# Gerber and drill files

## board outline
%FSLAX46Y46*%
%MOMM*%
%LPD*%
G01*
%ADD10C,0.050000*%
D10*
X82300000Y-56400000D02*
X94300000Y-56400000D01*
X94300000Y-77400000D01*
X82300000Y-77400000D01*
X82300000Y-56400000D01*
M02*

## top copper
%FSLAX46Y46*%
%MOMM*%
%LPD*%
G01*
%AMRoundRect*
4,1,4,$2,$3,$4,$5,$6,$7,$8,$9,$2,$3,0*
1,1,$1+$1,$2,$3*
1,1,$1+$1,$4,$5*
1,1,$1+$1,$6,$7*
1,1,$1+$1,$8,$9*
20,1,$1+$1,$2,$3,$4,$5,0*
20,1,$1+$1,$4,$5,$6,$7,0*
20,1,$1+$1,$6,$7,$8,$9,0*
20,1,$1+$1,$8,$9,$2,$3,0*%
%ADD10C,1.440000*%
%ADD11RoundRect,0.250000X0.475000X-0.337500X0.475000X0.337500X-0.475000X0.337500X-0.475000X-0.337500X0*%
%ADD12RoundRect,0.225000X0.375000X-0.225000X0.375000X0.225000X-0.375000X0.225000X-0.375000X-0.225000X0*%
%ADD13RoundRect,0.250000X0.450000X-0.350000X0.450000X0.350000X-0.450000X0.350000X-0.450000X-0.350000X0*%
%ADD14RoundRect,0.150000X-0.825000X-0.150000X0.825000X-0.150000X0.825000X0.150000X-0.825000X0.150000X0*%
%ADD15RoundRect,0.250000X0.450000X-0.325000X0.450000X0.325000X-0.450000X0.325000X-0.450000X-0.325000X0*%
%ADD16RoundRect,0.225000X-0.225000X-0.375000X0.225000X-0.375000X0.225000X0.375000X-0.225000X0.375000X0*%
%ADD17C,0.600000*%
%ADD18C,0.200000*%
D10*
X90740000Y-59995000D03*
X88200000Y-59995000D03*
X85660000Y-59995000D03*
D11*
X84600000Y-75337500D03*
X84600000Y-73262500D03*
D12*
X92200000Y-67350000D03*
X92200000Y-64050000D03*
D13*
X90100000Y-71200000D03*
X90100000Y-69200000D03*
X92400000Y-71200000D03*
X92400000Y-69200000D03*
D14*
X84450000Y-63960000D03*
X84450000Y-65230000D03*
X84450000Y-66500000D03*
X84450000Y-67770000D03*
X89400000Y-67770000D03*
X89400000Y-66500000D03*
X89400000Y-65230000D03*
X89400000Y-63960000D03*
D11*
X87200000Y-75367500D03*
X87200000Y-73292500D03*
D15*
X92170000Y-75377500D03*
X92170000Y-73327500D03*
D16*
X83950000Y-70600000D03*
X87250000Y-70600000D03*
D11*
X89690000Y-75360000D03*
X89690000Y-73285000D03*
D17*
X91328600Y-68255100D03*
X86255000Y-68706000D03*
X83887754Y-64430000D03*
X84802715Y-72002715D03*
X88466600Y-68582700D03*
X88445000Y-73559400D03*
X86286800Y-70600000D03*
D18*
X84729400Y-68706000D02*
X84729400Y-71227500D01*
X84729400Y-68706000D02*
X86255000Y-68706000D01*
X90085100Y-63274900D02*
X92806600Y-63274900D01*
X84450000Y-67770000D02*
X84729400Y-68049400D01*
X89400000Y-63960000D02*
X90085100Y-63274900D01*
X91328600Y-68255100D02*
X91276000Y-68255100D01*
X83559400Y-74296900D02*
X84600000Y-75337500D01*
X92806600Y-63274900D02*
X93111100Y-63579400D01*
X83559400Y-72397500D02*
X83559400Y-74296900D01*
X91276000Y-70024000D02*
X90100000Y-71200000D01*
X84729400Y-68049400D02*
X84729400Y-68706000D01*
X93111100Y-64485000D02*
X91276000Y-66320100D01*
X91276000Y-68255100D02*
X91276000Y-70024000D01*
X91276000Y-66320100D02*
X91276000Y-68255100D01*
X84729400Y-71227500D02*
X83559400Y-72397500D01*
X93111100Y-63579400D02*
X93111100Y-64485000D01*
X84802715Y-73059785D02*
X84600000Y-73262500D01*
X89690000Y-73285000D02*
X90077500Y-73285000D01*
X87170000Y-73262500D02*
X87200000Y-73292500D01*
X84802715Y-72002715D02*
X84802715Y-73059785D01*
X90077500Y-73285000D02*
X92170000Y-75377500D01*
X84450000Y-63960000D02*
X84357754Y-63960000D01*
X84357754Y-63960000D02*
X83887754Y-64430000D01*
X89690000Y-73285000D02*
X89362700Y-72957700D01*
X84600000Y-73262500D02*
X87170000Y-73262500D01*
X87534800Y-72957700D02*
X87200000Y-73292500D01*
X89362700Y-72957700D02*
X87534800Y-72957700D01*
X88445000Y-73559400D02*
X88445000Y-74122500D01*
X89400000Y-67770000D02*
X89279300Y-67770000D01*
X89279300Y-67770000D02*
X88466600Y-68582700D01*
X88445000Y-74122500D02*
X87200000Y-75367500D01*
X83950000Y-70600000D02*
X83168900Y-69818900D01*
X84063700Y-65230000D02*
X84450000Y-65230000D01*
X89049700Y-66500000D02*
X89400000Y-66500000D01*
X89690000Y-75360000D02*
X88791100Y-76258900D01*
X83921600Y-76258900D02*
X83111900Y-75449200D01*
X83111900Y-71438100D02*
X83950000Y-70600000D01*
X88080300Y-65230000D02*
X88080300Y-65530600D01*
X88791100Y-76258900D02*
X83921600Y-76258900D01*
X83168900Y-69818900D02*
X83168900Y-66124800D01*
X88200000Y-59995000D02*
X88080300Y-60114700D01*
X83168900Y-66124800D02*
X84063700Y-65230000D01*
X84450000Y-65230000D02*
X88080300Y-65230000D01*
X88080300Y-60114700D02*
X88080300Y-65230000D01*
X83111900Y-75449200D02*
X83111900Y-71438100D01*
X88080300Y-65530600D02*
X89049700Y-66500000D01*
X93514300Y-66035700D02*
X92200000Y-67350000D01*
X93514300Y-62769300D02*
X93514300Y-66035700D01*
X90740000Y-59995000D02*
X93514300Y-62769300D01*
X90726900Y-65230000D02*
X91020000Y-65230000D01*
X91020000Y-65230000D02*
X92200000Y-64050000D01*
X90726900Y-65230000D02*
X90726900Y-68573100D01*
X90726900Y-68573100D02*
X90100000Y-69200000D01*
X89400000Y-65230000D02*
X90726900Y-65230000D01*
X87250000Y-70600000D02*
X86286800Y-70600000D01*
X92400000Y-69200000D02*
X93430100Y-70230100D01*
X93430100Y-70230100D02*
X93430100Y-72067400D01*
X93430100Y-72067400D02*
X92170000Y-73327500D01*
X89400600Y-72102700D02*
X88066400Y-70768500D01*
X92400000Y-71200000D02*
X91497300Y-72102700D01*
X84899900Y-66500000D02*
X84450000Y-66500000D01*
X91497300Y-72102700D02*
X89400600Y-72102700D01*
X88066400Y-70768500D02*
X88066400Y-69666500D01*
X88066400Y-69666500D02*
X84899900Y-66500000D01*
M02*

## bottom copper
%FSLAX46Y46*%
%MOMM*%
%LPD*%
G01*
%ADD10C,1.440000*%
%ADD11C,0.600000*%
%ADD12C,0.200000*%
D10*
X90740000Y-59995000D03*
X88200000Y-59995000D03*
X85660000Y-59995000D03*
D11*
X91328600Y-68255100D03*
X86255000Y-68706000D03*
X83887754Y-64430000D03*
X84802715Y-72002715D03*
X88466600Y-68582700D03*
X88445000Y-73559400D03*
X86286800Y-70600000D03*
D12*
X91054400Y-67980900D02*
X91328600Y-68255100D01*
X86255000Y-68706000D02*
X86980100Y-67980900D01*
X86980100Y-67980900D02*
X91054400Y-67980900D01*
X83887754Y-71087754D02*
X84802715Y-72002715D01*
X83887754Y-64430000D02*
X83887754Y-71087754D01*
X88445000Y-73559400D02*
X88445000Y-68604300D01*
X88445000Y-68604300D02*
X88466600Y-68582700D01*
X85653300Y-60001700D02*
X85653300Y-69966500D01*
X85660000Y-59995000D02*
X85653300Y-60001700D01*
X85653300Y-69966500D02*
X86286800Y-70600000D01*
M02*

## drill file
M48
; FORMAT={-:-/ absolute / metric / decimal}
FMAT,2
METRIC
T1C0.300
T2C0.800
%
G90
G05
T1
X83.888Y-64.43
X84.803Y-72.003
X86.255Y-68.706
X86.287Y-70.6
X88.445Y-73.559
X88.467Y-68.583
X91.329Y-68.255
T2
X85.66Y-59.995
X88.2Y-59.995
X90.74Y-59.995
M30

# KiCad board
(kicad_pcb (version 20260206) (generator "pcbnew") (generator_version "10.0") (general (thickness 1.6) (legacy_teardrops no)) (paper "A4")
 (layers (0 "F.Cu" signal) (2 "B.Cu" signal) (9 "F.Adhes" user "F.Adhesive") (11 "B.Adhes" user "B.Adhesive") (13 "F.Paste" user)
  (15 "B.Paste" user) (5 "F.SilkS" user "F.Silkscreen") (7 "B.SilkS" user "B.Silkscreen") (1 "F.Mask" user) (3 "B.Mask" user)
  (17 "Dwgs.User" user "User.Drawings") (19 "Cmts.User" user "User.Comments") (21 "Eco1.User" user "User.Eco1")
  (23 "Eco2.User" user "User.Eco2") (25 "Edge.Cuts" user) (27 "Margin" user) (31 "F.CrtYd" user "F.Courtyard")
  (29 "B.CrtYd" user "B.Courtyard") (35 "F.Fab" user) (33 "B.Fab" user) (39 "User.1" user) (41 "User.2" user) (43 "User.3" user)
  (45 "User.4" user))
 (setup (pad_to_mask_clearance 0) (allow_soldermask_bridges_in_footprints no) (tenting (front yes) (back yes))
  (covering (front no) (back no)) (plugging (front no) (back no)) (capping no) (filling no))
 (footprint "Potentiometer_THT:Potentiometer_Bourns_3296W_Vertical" (layer "F.Cu") (at 90.74 59.995)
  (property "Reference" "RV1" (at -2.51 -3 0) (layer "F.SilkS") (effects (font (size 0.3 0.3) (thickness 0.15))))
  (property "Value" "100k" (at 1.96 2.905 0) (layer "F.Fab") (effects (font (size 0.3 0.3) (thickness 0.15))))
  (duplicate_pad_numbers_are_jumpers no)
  (pad "1" thru_hole circle (at 0 0) (size 1.44 1.44) (drill 0.8) (layers "*.Cu" "*.Mask") (remove_unused_layers no) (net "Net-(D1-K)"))
  (pad "2" thru_hole circle (at -2.54 0) (size 1.44 1.44) (drill 0.8) (layers "*.Cu" "*.Mask") (remove_unused_layers no) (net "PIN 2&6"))
  (pad "3" thru_hole circle (at -5.08 0) (size 1.44 1.44) (drill 0.8) (layers "*.Cu" "*.Mask") (remove_unused_layers no) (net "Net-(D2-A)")))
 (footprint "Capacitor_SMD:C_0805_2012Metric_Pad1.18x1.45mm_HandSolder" (layer "F.Cu") (at 84.6 74.3 90)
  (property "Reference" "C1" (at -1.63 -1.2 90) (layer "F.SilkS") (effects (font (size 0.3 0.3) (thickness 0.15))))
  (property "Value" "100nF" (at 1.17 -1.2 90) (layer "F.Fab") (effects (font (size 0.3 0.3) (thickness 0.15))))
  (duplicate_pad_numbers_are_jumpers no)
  (pad "1" smd roundrect (at -1.0375 0 90) (size 1.175 1.45) (layers "F.Cu" "F.Mask" "F.Paste") (roundrect_rratio 0.212766) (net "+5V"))
  (pad "2" smd roundrect (at 1.0375 0 90) (size 1.175 1.45) (layers "F.Cu" "F.Mask" "F.Paste") (roundrect_rratio 0.212766) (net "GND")))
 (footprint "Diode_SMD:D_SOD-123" (layer "F.Cu") (at 92.2 65.7 90)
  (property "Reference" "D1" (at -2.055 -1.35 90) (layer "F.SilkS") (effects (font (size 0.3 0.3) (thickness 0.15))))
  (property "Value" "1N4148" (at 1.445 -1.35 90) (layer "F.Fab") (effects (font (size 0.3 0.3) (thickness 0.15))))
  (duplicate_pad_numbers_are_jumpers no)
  (pad "1" smd roundrect (at -1.65 0 90) (size 0.9 1.2) (layers "F.Cu" "F.Mask" "F.Paste") (roundrect_rratio 0.25) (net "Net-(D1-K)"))
  (pad "2" smd roundrect (at 1.65 0 90) (size 0.9 1.2) (layers "F.Cu" "F.Mask" "F.Paste") (roundrect_rratio 0.25) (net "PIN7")))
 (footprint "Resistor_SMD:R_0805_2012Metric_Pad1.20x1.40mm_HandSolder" (layer "F.Cu") (at 90.1 70.2 90)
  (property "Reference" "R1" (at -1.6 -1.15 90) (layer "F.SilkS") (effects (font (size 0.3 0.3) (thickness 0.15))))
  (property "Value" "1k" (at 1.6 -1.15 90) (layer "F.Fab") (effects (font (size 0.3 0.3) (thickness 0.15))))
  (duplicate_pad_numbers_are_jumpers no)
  (pad "1" smd roundrect (at -1 0 90) (size 1.2 1.4) (layers "F.Cu" "F.Mask" "F.Paste") (roundrect_rratio 0.208333) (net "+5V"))
  (pad "2" smd roundrect (at 1 0 90) (size 1.2 1.4) (layers "F.Cu" "F.Mask" "F.Paste") (roundrect_rratio 0.208333) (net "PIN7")))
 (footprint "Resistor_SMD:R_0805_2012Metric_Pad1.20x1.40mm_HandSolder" (layer "F.Cu") (at 92.4 70.2 90)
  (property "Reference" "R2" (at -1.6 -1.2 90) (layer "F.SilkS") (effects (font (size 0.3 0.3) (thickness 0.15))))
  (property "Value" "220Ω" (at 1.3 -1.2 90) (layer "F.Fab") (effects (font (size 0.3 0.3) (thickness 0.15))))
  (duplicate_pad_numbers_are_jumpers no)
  (pad "1" smd roundrect (at -1 0 90) (size 1.2 1.4) (layers "F.Cu" "F.Mask" "F.Paste") (roundrect_rratio 0.208333) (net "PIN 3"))
  (pad "2" smd roundrect (at 1 0 90) (size 1.2 1.4) (layers "F.Cu" "F.Mask" "F.Paste") (roundrect_rratio 0.208333) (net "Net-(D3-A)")))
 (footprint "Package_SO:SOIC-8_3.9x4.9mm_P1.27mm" (layer "F.Cu") (at 86.925 65.865)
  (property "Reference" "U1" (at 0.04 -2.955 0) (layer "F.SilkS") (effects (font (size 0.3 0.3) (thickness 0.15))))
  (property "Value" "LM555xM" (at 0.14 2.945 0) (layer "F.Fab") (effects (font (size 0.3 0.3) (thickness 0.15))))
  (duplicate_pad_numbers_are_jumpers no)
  (pad "1" smd roundrect (at -2.475 -1.905) (size 1.95 0.6) (layers "F.Cu" "F.Mask" "F.Paste") (roundrect_rratio 0.25) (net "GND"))
  (pad "2" smd roundrect (at -2.475 -0.635) (size 1.95 0.6) (layers "F.Cu" "F.Mask" "F.Paste") (roundrect_rratio 0.25) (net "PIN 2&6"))
  (pad "3" smd roundrect (at -2.475 0.635) (size 1.95 0.6) (layers "F.Cu" "F.Mask" "F.Paste") (roundrect_rratio 0.25) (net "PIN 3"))
  (pad "4" smd roundrect (at -2.475 1.905) (size 1.95 0.6) (layers "F.Cu" "F.Mask" "F.Paste") (roundrect_rratio 0.25) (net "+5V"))
  (pad "5" smd roundrect (at 2.475 1.905) (size 1.95 0.6) (layers "F.Cu" "F.Mask" "F.Paste") (roundrect_rratio 0.25) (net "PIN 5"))
  (pad "6" smd roundrect (at 2.475 0.635) (size 1.95 0.6) (layers "F.Cu" "F.Mask" "F.Paste") (roundrect_rratio 0.25) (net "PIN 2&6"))
  (pad "7" smd roundrect (at 2.475 -0.635) (size 1.95 0.6) (layers "F.Cu" "F.Mask" "F.Paste") (roundrect_rratio 0.25) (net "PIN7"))
  (pad "8" smd roundrect (at 2.475 -1.905) (size 1.95 0.6) (layers "F.Cu" "F.Mask" "F.Paste") (roundrect_rratio 0.25) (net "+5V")))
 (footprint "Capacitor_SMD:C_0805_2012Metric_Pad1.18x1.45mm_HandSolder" (layer "F.Cu") (at 87.2 74.33 90)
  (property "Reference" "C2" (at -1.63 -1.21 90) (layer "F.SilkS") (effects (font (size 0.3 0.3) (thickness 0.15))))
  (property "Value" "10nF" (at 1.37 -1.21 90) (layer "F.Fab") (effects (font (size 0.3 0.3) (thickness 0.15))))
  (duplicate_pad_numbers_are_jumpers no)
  (pad "1" smd roundrect (at -1.0375 0 90) (size 1.175 1.45) (layers "F.Cu" "F.Mask" "F.Paste") (roundrect_rratio 0.212766) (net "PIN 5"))
  (pad "2" smd roundrect (at 1.0375 0 90) (size 1.175 1.45) (layers "F.Cu" "F.Mask" "F.Paste") (roundrect_rratio 0.212766) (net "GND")))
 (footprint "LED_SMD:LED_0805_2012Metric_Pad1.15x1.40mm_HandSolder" (layer "F.Cu") (at 92.17 74.3525 90)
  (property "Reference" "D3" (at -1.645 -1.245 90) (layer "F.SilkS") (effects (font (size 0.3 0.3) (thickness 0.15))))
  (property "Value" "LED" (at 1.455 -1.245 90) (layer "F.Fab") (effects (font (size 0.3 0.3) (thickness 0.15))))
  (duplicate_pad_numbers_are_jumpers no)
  (pad "1" smd roundrect (at -1.025 0 90) (size 1.15 1.4) (layers "F.Cu" "F.Mask" "F.Paste") (roundrect_rratio 0.217391) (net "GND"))
  (pad "2" smd roundrect (at 1.025 0 90) (size 1.15 1.4) (layers "F.Cu" "F.Mask" "F.Paste") (roundrect_rratio 0.217391) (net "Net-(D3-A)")))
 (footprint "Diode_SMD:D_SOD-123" (layer "F.Cu") (at 85.6 70.6)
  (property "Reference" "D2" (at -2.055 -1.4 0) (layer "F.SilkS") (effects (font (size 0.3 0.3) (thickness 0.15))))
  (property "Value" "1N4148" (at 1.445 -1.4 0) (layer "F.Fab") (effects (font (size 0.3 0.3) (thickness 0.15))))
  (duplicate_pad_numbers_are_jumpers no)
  (pad "1" smd roundrect (at -1.65 0) (size 0.9 1.2) (layers "F.Cu" "F.Mask" "F.Paste") (roundrect_rratio 0.25) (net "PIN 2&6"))
  (pad "2" smd roundrect (at 1.65 0) (size 0.9 1.2) (layers "F.Cu" "F.Mask" "F.Paste") (roundrect_rratio 0.25) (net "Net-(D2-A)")))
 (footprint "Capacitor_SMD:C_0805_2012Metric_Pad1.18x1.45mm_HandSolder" (layer "F.Cu") (at 89.69 74.3225 90)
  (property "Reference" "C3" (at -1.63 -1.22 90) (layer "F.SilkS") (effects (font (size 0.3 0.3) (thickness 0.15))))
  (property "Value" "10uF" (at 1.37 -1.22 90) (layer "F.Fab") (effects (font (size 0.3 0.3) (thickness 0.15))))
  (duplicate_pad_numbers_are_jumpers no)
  (pad "1" smd roundrect (at -1.0375 0 90) (size 1.175 1.45) (layers "F.Cu" "F.Mask" "F.Paste") (roundrect_rratio 0.212766) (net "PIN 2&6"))
  (pad "2" smd roundrect (at 1.0375 0 90) (size 1.175 1.45) (layers "F.Cu" "F.Mask" "F.Paste") (roundrect_rratio 0.212766) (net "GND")))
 (gr_rect (start 82.3 56.4) (end 94.3 77.4) (stroke (width 0.05) (type default)) (fill no) (layer "Edge.Cuts"))
 (segment (start 84.7294 68.706) (end 84.7294 71.2275) (width 0.2) (layer "F.Cu") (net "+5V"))
 (segment (start 84.7294 68.706) (end 86.255 68.706) (width 0.2) (layer "F.Cu") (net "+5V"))
 (segment (start 90.0851 63.2749) (end 92.8066 63.2749) (width 0.2) (layer "F.Cu") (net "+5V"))
 (segment (start 84.45 67.77) (end 84.7294 68.0494) (width 0.2) (layer "F.Cu") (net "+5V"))
 (segment (start 89.4 63.96) (end 90.0851 63.2749) (width 0.2) (layer "F.Cu") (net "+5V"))
 (segment (start 91.3286 68.2551) (end 91.276 68.2551) (width 0.2) (layer "F.Cu") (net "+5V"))
 (segment (start 83.5594 74.2969) (end 84.6 75.3375) (width 0.2) (layer "F.Cu") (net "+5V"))
 (segment (start 92.8066 63.2749) (end 93.1111 63.5794) (width 0.2) (layer "F.Cu") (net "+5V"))
 (segment (start 83.5594 72.3975) (end 83.5594 74.2969) (width 0.2) (layer "F.Cu") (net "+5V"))
 (segment (start 91.276 70.024) (end 90.1 71.2) (width 0.2) (layer "F.Cu") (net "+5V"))
 (segment (start 84.7294 68.0494) (end 84.7294 68.706) (width 0.2) (layer "F.Cu") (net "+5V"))
 (segment (start 93.1111 64.485) (end 91.276 66.3201) (width 0.2) (layer "F.Cu") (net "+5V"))
 (segment (start 91.276 68.2551) (end 91.276 70.024) (width 0.2) (layer "F.Cu") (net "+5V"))
 (segment (start 91.276 66.3201) (end 91.276 68.2551) (width 0.2) (layer "F.Cu") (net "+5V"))
 (segment (start 84.7294 71.2275) (end 83.5594 72.3975) (width 0.2) (layer "F.Cu") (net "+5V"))
 (segment (start 93.1111 63.5794) (end 93.1111 64.485) (width 0.2) (layer "F.Cu") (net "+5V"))
 (via (at 91.3286 68.2551) (size 0.6) (drill 0.3) (layers "F.Cu" "B.Cu") (capping no) (covering (front no) (back no))
  (plugging (front no) (back no)) (filling no) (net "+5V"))
 (via (at 86.255 68.706) (size 0.6) (drill 0.3) (layers "F.Cu" "B.Cu") (capping no) (covering (front no) (back no))
  (plugging (front no) (back no)) (filling no) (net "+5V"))
 (segment (start 91.0544 67.9809) (end 91.3286 68.2551) (width 0.2) (layer "B.Cu") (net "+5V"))
 (segment (start 86.255 68.706) (end 86.9801 67.9809) (width 0.2) (layer "B.Cu") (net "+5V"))
 (segment (start 86.9801 67.9809) (end 91.0544 67.9809) (width 0.2) (layer "B.Cu") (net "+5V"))
 (segment (start 84.802715 73.059785) (end 84.6 73.2625) (width 0.2) (layer "F.Cu") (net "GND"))
 (segment (start 89.69 73.285) (end 90.0775 73.285) (width 0.2) (layer "F.Cu") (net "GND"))
 (segment (start 87.17 73.2625) (end 87.2 73.2925) (width 0.2) (layer "F.Cu") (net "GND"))
 (segment (start 84.802715 72.002715) (end 84.802715 73.059785) (width 0.2) (layer "F.Cu") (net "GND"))
 (segment (start 90.0775 73.285) (end 92.17 75.3775) (width 0.2) (layer "F.Cu") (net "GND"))
 (segment (start 84.45 63.96) (end 84.357754 63.96) (width 0.2) (layer "F.Cu") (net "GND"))
 (segment (start 84.357754 63.96) (end 83.887754 64.43) (width 0.2) (layer "F.Cu") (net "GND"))
 (segment (start 89.69 73.285) (end 89.3627 72.9577) (width 0.2) (layer "F.Cu") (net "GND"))
 (segment (start 84.6 73.2625) (end 87.17 73.2625) (width 0.2) (layer "F.Cu") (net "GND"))
 (segment (start 87.5348 72.9577) (end 87.2 73.2925) (width 0.2) (layer "F.Cu") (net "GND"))
 (segment (start 89.3627 72.9577) (end 87.5348 72.9577) (width 0.2) (layer "F.Cu") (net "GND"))
 (via (at 83.887754 64.43) (size 0.6) (drill 0.3) (layers "F.Cu" "B.Cu") (capping no) (covering (front no) (back no))
  (plugging (front no) (back no)) (filling no) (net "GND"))
 (via (at 84.802715 72.002715) (size 0.6) (drill 0.3) (layers "F.Cu" "B.Cu") (capping no) (covering (front no) (back no))
  (plugging (front no) (back no)) (filling no) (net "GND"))
 (segment (start 83.887754 71.087754) (end 84.802715 72.002715) (width 0.2) (layer "B.Cu") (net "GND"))
 (segment (start 83.887754 64.43) (end 83.887754 71.087754) (width 0.2) (layer "B.Cu") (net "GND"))
 (segment (start 88.445 73.5594) (end 88.445 74.1225) (width 0.2) (layer "F.Cu") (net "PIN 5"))
 (segment (start 89.4 67.77) (end 89.2793 67.77) (width 0.2) (layer "F.Cu") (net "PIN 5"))
 (segment (start 89.2793 67.77) (end 88.4666 68.5827) (width 0.2) (layer "F.Cu") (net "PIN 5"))
 (segment (start 88.445 74.1225) (end 87.2 75.3675) (width 0.2) (layer "F.Cu") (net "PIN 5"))
 (via (at 88.4666 68.5827) (size 0.6) (drill 0.3) (layers "F.Cu" "B.Cu") (capping no) (covering (front no) (back no))
  (plugging (front no) (back no)) (filling no) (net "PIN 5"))
 (via (at 88.445 73.5594) (size 0.6) (drill 0.3) (layers "F.Cu" "B.Cu") (capping no) (covering (front no) (back no))
  (plugging (front no) (back no)) (filling no) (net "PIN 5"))
 (segment (start 88.445 73.5594) (end 88.445 68.6043) (width 0.2) (layer "B.Cu") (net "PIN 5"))
 (segment (start 88.445 68.6043) (end 88.4666 68.5827) (width 0.2) (layer "B.Cu") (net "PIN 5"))
 (segment (start 83.95 70.6) (end 83.1689 69.8189) (width 0.2) (layer "F.Cu") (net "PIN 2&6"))
 (segment (start 84.0637 65.23) (end 84.45 65.23) (width 0.2) (layer "F.Cu") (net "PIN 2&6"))
 (segment (start 89.0497 66.5) (end 89.4 66.5) (width 0.2) (layer "F.Cu") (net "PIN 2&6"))
 (segment (start 89.69 75.36) (end 88.7911 76.2589) (width 0.2) (layer "F.Cu") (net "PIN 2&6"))
 (segment (start 83.9216 76.2589) (end 83.1119 75.4492) (width 0.2) (layer "F.Cu") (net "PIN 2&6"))
 (segment (start 83.1119 71.4381) (end 83.95 70.6) (width 0.2) (layer "F.Cu") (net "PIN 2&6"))
 (segment (start 88.0803 65.23) (end 88.0803 65.5306) (width 0.2) (layer "F.Cu") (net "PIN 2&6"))
 (segment (start 88.7911 76.2589) (end 83.9216 76.2589) (width 0.2) (layer "F.Cu") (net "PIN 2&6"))
 (segment (start 83.1689 69.8189) (end 83.1689 66.1248) (width 0.2) (layer "F.Cu") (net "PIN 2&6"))
 (segment (start 88.2 59.995) (end 88.0803 60.1147) (width 0.2) (layer "F.Cu") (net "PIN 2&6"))
 (segment (start 83.1689 66.1248) (end 84.0637 65.23) (width 0.2) (layer "F.Cu") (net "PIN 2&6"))
 (segment (start 84.45 65.23) (end 88.0803 65.23) (width 0.2) (layer "F.Cu") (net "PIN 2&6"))
 (segment (start 88.0803 60.1147) (end 88.0803 65.23) (width 0.2) (layer "F.Cu") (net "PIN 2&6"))
 (segment (start 83.1119 75.4492) (end 83.1119 71.4381) (width 0.2) (layer "F.Cu") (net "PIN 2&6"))
 (segment (start 88.0803 65.5306) (end 89.0497 66.5) (width 0.2) (layer "F.Cu") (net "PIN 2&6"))
 (segment (start 93.5143 66.0357) (end 92.2 67.35) (width 0.2) (layer "F.Cu") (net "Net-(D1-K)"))
 (segment (start 93.5143 62.7693) (end 93.5143 66.0357) (width 0.2) (layer "F.Cu") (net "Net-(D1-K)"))
 (segment (start 90.74 59.995) (end 93.5143 62.7693) (width 0.2) (layer "F.Cu") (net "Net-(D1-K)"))
 (segment (start 90.7269 65.23) (end 91.02 65.23) (width 0.2) (layer "F.Cu") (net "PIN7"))
 (segment (start 91.02 65.23) (end 92.2 64.05) (width 0.2) (layer "F.Cu") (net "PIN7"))
 (segment (start 90.7269 65.23) (end 90.7269 68.5731) (width 0.2) (layer "F.Cu") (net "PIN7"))
 (segment (start 90.7269 68.5731) (end 90.1 69.2) (width 0.2) (layer "F.Cu") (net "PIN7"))
 (segment (start 89.4 65.23) (end 90.7269 65.23) (width 0.2) (layer "F.Cu") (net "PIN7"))
 (segment (start 87.25 70.6) (end 86.2868 70.6) (width 0.2) (layer "F.Cu") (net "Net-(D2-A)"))
 (via (at 86.2868 70.6) (size 0.6) (drill 0.3) (layers "F.Cu" "B.Cu") (capping no) (covering (front no) (back no))
  (plugging (front no) (back no)) (filling no) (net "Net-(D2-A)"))
 (segment (start 85.6533 60.0017) (end 85.6533 69.9665) (width 0.2) (layer "B.Cu") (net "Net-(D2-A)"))
 (segment (start 85.66 59.995) (end 85.6533 60.0017) (width 0.2) (layer "B.Cu") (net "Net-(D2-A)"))
 (segment (start 85.6533 69.9665) (end 86.2868 70.6) (width 0.2) (layer "B.Cu") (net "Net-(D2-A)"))
 (segment (start 92.4 69.2) (end 93.4301 70.2301) (width 0.2) (layer "F.Cu") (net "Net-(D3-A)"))
 (segment (start 93.4301 70.2301) (end 93.4301 72.0674) (width 0.2) (layer "F.Cu") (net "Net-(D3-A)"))
 (segment (start 93.4301 72.0674) (end 92.17 73.3275) (width 0.2) (layer "F.Cu") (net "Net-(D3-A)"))
 (segment (start 89.4006 72.1027) (end 88.0664 70.7685) (width 0.2) (layer "F.Cu") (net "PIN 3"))
 (segment (start 92.4 71.2) (end 91.4973 72.1027) (width 0.2) (layer "F.Cu") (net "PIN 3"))
 (segment (start 84.8999 66.5) (end 84.45 66.5) (width 0.2) (layer "F.Cu") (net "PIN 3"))
 (segment (start 91.4973 72.1027) (end 89.4006 72.1027) (width 0.2) (layer "F.Cu") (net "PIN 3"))
 (segment (start 88.0664 70.7685) (end 88.0664 69.6665) (width 0.2) (layer "F.Cu") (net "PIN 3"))
 (segment (start 88.0664 69.6665) (end 84.8999 66.5) (width 0.2) (layer "F.Cu") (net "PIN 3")))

